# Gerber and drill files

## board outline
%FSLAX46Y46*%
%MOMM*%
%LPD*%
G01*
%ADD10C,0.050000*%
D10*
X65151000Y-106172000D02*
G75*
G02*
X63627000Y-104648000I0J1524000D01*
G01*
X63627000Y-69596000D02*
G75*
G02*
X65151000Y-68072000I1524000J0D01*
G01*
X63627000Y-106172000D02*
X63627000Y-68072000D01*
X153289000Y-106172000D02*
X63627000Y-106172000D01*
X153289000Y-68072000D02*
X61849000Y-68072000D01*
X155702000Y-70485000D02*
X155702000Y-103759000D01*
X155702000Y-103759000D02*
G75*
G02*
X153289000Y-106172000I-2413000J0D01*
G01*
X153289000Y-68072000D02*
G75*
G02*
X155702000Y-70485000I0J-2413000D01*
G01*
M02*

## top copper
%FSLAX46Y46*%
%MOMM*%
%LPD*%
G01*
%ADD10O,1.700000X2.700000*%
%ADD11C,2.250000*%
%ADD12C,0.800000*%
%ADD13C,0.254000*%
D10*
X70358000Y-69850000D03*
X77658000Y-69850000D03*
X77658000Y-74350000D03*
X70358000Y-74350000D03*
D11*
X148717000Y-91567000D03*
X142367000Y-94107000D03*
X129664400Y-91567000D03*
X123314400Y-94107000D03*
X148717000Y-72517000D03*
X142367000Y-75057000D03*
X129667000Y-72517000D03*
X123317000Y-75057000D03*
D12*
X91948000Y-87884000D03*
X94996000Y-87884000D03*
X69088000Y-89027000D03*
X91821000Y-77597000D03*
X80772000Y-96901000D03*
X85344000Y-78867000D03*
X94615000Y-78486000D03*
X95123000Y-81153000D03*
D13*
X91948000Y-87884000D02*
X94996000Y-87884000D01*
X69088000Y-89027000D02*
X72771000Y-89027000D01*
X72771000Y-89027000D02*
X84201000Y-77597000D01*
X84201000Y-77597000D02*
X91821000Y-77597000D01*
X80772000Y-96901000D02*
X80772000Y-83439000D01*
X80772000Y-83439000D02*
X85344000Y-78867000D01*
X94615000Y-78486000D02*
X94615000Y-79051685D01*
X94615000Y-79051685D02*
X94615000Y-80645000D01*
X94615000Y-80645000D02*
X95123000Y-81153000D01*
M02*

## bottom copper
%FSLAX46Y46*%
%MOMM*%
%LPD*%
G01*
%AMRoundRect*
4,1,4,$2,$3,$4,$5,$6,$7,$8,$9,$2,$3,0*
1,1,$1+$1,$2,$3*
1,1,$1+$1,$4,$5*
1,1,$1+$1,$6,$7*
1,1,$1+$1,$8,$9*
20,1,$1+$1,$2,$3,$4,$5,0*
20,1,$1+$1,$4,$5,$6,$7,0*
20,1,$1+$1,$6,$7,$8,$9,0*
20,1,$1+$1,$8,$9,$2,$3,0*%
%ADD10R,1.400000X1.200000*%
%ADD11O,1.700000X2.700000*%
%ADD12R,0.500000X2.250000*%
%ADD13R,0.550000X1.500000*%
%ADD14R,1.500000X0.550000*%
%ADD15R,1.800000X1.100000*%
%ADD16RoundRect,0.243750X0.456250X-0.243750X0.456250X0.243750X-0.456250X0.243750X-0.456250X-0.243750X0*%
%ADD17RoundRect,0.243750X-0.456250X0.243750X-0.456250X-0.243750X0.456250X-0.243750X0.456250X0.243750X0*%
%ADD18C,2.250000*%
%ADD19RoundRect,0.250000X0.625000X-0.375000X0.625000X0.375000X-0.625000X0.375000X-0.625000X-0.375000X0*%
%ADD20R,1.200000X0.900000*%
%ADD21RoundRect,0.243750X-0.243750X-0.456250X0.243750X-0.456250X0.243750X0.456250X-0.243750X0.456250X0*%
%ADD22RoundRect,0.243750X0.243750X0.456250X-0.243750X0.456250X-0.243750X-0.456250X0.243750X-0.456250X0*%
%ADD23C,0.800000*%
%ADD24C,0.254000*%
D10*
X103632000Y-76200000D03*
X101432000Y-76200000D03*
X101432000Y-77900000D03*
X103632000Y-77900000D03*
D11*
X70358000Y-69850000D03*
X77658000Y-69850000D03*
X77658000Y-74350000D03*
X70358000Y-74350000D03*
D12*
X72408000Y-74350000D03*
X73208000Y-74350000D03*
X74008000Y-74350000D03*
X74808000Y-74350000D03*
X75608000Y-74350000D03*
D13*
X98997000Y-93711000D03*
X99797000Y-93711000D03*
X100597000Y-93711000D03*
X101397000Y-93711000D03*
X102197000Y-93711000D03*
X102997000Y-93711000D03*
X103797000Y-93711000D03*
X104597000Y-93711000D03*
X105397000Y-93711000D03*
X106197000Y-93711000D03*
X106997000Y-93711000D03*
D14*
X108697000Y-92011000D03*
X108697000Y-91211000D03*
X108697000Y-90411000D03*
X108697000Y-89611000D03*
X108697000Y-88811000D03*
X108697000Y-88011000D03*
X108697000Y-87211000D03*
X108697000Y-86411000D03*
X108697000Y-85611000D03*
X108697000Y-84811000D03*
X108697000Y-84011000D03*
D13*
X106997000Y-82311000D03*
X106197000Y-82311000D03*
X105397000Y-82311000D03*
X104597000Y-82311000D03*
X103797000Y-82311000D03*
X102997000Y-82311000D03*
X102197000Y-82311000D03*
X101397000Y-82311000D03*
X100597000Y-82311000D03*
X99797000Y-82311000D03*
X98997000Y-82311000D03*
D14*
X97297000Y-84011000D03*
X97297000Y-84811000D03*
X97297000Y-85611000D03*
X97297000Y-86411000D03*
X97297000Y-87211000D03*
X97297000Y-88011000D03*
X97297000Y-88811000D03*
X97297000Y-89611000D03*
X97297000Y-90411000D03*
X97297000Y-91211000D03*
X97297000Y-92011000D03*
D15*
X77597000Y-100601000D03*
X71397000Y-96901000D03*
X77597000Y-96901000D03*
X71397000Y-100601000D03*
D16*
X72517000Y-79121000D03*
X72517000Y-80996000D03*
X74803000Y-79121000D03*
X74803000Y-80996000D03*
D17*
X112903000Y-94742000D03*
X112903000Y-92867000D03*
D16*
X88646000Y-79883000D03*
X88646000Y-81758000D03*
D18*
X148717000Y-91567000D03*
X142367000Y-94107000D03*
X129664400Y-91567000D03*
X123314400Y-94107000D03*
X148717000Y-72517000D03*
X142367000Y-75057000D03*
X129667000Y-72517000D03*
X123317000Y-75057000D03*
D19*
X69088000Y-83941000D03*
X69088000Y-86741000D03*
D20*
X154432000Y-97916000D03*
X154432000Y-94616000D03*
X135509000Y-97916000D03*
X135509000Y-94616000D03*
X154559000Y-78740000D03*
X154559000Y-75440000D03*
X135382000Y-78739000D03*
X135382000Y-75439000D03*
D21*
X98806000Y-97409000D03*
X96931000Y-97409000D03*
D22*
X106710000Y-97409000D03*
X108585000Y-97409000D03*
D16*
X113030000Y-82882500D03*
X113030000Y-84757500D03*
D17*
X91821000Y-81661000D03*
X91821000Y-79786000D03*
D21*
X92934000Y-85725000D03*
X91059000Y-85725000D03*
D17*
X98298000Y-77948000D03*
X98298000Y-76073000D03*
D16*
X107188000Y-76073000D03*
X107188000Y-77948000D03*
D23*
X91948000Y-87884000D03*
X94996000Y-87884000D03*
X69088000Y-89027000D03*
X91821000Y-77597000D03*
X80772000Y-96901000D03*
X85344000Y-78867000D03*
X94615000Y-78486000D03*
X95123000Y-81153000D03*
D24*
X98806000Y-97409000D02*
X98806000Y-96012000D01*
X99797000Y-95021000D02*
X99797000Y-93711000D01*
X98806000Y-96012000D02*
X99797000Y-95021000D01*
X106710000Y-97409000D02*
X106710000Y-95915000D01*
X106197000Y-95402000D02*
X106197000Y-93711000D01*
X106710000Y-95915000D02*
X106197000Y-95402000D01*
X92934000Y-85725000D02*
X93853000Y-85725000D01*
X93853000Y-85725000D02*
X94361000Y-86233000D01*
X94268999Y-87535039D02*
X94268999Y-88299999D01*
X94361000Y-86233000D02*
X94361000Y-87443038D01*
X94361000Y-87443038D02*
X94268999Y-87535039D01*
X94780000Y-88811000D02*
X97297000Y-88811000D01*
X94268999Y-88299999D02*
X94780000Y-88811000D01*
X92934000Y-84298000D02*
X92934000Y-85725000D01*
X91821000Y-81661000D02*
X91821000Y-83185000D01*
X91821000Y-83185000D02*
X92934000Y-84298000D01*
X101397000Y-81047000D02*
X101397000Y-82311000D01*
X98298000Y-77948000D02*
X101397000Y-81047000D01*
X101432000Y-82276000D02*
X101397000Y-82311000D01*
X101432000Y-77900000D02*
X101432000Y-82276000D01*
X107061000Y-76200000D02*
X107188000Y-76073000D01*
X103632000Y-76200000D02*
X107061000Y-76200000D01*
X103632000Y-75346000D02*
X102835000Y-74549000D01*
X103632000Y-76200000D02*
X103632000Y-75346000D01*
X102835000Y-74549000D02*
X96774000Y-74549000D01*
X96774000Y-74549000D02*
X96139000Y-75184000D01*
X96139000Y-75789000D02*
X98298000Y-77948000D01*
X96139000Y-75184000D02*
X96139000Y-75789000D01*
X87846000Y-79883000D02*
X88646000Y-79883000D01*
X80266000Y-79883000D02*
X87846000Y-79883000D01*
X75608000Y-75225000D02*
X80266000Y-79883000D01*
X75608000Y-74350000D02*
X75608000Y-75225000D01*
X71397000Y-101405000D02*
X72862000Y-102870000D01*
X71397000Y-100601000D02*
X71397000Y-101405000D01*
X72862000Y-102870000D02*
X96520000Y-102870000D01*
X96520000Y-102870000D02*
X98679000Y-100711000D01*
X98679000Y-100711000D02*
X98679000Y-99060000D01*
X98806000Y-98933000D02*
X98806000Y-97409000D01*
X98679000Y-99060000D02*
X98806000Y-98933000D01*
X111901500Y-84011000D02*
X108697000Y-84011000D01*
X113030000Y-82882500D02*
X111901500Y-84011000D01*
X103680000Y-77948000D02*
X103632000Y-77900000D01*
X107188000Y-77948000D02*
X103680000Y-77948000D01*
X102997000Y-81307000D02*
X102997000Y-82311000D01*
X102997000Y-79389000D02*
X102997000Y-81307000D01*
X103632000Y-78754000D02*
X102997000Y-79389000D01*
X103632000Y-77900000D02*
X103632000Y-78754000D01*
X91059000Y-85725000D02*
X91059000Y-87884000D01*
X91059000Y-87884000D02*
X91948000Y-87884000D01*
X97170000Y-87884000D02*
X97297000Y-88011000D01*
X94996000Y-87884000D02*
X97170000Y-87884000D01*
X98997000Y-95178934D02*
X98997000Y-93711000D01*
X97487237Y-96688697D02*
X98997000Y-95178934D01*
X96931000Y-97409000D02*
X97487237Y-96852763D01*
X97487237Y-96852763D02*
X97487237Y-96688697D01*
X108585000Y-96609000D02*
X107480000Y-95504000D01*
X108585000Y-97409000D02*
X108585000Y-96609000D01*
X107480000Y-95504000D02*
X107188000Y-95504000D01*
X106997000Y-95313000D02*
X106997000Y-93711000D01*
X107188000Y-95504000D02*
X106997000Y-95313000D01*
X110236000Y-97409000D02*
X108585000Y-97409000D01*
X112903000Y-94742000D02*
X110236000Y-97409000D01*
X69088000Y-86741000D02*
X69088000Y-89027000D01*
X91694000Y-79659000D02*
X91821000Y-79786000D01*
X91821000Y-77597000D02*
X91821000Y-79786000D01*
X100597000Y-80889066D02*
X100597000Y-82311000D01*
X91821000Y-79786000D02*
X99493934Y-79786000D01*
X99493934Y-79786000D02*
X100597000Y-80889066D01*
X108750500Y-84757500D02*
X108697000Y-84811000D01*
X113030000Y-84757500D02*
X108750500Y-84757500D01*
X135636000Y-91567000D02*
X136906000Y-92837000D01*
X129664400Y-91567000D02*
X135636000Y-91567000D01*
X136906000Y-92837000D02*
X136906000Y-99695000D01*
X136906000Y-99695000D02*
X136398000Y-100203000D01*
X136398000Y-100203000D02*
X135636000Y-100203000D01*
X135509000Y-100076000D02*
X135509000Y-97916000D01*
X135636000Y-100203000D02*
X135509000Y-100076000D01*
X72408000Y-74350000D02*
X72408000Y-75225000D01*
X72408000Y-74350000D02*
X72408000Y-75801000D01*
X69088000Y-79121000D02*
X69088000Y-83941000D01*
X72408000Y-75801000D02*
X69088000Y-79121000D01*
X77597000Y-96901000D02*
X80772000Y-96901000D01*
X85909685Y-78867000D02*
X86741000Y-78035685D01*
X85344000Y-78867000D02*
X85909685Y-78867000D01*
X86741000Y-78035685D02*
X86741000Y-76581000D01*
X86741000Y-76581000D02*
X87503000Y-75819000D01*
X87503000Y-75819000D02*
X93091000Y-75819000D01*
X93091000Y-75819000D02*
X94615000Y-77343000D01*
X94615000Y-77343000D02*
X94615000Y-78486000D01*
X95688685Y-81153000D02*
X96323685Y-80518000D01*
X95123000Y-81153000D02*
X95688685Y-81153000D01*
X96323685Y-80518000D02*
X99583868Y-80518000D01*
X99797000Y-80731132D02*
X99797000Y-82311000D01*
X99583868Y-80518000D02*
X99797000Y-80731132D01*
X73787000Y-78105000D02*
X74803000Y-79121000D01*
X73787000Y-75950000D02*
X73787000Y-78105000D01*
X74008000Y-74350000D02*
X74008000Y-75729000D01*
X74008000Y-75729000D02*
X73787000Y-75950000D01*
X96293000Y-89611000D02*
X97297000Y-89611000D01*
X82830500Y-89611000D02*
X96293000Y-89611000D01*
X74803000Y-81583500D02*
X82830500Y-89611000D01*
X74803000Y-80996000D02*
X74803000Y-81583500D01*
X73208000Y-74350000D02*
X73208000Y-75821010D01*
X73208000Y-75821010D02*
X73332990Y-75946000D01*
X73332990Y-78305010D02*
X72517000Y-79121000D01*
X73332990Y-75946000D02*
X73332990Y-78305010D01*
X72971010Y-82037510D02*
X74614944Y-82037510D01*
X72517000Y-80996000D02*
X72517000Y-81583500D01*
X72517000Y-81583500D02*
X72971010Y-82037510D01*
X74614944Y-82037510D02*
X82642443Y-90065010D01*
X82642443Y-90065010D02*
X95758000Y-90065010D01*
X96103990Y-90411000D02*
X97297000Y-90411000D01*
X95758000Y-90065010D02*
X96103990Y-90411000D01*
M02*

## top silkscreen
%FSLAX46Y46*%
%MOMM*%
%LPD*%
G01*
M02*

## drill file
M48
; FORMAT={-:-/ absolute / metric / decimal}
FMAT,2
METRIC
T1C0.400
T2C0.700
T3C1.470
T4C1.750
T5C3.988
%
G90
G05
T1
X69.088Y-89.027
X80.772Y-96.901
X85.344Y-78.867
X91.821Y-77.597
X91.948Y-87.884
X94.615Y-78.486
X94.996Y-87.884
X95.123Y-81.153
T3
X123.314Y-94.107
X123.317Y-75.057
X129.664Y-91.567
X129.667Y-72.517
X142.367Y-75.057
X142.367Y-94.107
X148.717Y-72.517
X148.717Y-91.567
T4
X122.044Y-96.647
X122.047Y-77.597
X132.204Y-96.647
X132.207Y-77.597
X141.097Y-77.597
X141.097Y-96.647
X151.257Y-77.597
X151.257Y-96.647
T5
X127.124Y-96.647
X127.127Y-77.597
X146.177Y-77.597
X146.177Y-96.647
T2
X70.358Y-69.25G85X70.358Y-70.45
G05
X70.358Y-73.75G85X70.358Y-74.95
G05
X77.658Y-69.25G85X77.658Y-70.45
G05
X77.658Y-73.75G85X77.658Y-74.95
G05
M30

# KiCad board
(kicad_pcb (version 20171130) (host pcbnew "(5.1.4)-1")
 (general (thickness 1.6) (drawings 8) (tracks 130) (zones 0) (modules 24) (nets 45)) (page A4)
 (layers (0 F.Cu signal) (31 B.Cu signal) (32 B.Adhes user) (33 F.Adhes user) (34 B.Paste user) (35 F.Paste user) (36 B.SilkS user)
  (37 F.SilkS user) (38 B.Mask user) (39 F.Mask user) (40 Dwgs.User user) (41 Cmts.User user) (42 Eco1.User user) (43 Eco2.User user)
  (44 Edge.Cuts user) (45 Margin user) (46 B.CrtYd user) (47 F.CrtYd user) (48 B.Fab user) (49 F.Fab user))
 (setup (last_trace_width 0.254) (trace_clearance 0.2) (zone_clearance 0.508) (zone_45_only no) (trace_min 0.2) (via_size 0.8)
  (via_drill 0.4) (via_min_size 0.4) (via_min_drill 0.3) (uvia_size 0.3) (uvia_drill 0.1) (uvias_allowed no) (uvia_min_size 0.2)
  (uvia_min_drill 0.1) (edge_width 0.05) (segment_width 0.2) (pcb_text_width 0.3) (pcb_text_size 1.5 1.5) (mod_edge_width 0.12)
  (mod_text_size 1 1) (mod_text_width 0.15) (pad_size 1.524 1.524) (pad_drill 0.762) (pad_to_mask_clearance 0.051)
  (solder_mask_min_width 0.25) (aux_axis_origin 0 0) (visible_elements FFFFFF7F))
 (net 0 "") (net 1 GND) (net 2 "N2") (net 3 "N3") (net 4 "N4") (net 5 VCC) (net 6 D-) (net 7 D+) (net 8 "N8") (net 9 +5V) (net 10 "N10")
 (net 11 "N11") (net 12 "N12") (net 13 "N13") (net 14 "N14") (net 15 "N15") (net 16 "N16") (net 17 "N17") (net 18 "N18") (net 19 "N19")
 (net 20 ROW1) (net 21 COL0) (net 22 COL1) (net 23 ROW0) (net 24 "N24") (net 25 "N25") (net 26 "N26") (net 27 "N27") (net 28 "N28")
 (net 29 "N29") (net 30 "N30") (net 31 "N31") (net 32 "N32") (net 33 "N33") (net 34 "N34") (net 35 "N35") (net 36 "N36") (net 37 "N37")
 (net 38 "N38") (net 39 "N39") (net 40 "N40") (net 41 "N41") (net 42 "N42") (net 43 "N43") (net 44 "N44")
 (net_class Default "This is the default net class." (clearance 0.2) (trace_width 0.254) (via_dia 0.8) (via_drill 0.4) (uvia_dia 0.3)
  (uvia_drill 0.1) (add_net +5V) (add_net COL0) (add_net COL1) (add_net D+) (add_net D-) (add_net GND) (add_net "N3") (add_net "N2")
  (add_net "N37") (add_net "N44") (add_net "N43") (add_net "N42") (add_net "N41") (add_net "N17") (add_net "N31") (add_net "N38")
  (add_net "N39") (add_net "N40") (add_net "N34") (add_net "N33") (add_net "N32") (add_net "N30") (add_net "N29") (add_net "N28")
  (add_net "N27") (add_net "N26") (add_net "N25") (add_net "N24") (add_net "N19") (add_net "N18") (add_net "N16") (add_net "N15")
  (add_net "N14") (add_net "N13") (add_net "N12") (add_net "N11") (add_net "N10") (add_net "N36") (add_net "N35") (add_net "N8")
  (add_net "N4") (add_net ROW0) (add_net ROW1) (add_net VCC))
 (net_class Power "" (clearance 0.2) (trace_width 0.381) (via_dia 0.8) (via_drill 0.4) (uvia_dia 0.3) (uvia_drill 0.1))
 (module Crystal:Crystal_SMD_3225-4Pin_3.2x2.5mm (layer B.Cu) (at 102.532 77.05 180)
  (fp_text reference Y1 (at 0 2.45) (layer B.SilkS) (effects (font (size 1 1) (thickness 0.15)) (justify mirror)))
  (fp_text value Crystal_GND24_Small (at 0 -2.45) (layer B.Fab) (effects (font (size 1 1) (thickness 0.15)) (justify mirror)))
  (pad 4 smd rect (at -1.1 0.85 180) (size 1.4 1.2) (layers B.Cu B.Paste B.Mask) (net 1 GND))
  (pad 3 smd rect (at 1.1 0.85 180) (size 1.4 1.2) (layers B.Cu B.Paste B.Mask) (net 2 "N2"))
  (pad 2 smd rect (at 1.1 -0.85 180) (size 1.4 1.2) (layers B.Cu B.Paste B.Mask) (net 1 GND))
  (pad 1 smd rect (at -1.1 -0.85 180) (size 1.4 1.2) (layers B.Cu B.Paste B.Mask) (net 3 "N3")))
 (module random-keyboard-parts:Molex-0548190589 (layer B.Cu) (at 74.008 69.85 270)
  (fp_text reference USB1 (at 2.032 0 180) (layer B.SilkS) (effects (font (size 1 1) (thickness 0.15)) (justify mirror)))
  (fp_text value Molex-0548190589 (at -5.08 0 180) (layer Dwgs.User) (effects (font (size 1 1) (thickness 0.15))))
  (pad 6 thru_hole oval (at 0 3.65 270) (size 2.7 1.7) (drill oval 1.9 0.7) (layers *.Cu *.Mask) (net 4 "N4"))
  (pad 6 thru_hole oval (at 0 -3.65 270) (size 2.7 1.7) (drill oval 1.9 0.7) (layers *.Cu *.Mask) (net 4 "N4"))
  (pad 6 thru_hole oval (at 4.5 -3.65 270) (size 2.7 1.7) (drill oval 1.9 0.7) (layers *.Cu *.Mask) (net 4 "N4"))
  (pad 6 thru_hole oval (at 4.5 3.65 270) (size 2.7 1.7) (drill oval 1.9 0.7) (layers *.Cu *.Mask) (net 4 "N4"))
  (pad 5 smd rect (at 4.5 1.6 270) (size 2.25 0.5) (layers B.Cu B.Paste B.Mask) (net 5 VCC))
  (pad 4 smd rect (at 4.5 0.8 270) (size 2.25 0.5) (layers B.Cu B.Paste B.Mask) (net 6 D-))
  (pad 3 smd rect (at 4.5 0 270) (size 2.25 0.5) (layers B.Cu B.Paste B.Mask) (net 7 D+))
  (pad 2 smd rect (at 4.5 -0.8 270) (size 2.25 0.5) (layers B.Cu B.Paste B.Mask) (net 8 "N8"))
  (pad 1 smd rect (at 4.5 -1.6 270) (size 2.25 0.5) (layers B.Cu B.Paste B.Mask) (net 1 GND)))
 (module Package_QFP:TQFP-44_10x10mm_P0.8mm (layer B.Cu) (at 102.997 88.011)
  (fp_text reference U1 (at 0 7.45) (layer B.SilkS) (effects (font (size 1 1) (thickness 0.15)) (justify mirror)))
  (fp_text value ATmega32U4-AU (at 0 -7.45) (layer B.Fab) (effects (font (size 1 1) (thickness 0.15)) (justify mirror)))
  (pad 44 smd rect (at -4 5.7 270) (size 1.5 0.55) (layers B.Cu B.Paste B.Mask) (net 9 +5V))
  (pad 43 smd rect (at -3.2 5.7 270) (size 1.5 0.55) (layers B.Cu B.Paste B.Mask) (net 1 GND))
  (pad 42 smd rect (at -2.4 5.7 270) (size 1.5 0.55) (layers B.Cu B.Paste B.Mask) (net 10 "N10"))
  (pad 41 smd rect (at -1.6 5.7 270) (size 1.5 0.55) (layers B.Cu B.Paste B.Mask) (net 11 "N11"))
  (pad 40 smd rect (at -0.8 5.7 270) (size 1.5 0.55) (layers B.Cu B.Paste B.Mask) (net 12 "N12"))
  (pad 39 smd rect (at 0 5.7 270) (size 1.5 0.55) (layers B.Cu B.Paste B.Mask) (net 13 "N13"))
  (pad 38 smd rect (at 0.8 5.7 270) (size 1.5 0.55) (layers B.Cu B.Paste B.Mask) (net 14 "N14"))
  (pad 37 smd rect (at 1.6 5.7 270) (size 1.5 0.55) (layers B.Cu B.Paste B.Mask) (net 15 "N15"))
  (pad 36 smd rect (at 2.4 5.7 270) (size 1.5 0.55) (layers B.Cu B.Paste B.Mask) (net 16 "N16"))
  (pad 35 smd rect (at 3.2 5.7 270) (size 1.5 0.55) (layers B.Cu B.Paste B.Mask) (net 1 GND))
  (pad 34 smd rect (at 4 5.7 270) (size 1.5 0.55) (layers B.Cu B.Paste B.Mask) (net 9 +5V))
  (pad 33 smd rect (at 5.7 4) (size 1.5 0.55) (layers B.Cu B.Paste B.Mask) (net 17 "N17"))
  (pad 32 smd rect (at 5.7 3.2) (size 1.5 0.55) (layers B.Cu B.Paste B.Mask) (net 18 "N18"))
  (pad 31 smd rect (at 5.7 2.4) (size 1.5 0.55) (layers B.Cu B.Paste B.Mask) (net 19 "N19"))
  (pad 30 smd rect (at 5.7 1.6) (size 1.5 0.55) (layers B.Cu B.Paste B.Mask) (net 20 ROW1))
  (pad 29 smd rect (at 5.7 0.8) (size 1.5 0.55) (layers B.Cu B.Paste B.Mask) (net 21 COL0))
  (pad 28 smd rect (at 5.7 0) (size 1.5 0.55) (layers B.Cu B.Paste B.Mask) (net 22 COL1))
  (pad 27 smd rect (at 5.7 -0.8) (size 1.5 0.55) (layers B.Cu B.Paste B.Mask) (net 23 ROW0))
  (pad 26 smd rect (at 5.7 -1.6) (size 1.5 0.55) (layers B.Cu B.Paste B.Mask) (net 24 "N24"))
  (pad 25 smd rect (at 5.7 -2.4) (size 1.5 0.55) (layers B.Cu B.Paste B.Mask) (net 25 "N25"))
  (pad 24 smd rect (at 5.7 -3.2) (size 1.5 0.55) (layers B.Cu B.Paste B.Mask) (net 9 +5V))
  (pad 23 smd rect (at 5.7 -4) (size 1.5 0.55) (layers B.Cu B.Paste B.Mask) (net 1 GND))
  (pad 22 smd rect (at 4 -5.7 270) (size 1.5 0.55) (layers B.Cu B.Paste B.Mask) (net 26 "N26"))
  (pad 21 smd rect (at 3.2 -5.7 270) (size 1.5 0.55) (layers B.Cu B.Paste B.Mask) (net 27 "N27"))
  (pad 20 smd rect (at 2.4 -5.7 270) (size 1.5 0.55) (layers B.Cu B.Paste B.Mask) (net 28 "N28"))
  (pad 19 smd rect (at 1.6 -5.7 270) (size 1.5 0.55) (layers B.Cu B.Paste B.Mask) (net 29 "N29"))
  (pad 18 smd rect (at 0.8 -5.7 270) (size 1.5 0.55) (layers B.Cu B.Paste B.Mask) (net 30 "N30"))
  (pad 17 smd rect (at 0 -5.7 270) (size 1.5 0.55) (layers B.Cu B.Paste B.Mask) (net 3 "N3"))
  (pad 16 smd rect (at -0.8 -5.7 270) (size 1.5 0.55) (layers B.Cu B.Paste B.Mask) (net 2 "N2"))
  (pad 15 smd rect (at -1.6 -5.7 270) (size 1.5 0.55) (layers B.Cu B.Paste B.Mask) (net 1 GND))
  (pad 14 smd rect (at -2.4 -5.7 270) (size 1.5 0.55) (layers B.Cu B.Paste B.Mask) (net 9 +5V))
  (pad 13 smd rect (at -3.2 -5.7 270) (size 1.5 0.55) (layers B.Cu B.Paste B.Mask) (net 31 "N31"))
  (pad 12 smd rect (at -4 -5.7 270) (size 1.5 0.55) (layers B.Cu B.Paste B.Mask) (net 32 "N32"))
  (pad 11 smd rect (at -5.7 -4) (size 1.5 0.55) (layers B.Cu B.Paste B.Mask) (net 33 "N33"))
  (pad 10 smd rect (at -5.7 -3.2) (size 1.5 0.55) (layers B.Cu B.Paste B.Mask) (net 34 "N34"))
  (pad 9 smd rect (at -5.7 -2.4) (size 1.5 0.55) (layers B.Cu B.Paste B.Mask) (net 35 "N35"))
  (pad 8 smd rect (at -5.7 -1.6) (size 1.5 0.55) (layers B.Cu B.Paste B.Mask) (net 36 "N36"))
  (pad 7 smd rect (at -5.7 -0.8) (size 1.5 0.55) (layers B.Cu B.Paste B.Mask) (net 9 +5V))
  (pad 6 smd rect (at -5.7 0) (size 1.5 0.55) (layers B.Cu B.Paste B.Mask) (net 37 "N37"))
  (pad 5 smd rect (at -5.7 0.8) (size 1.5 0.55) (layers B.Cu B.Paste B.Mask) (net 1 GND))
  (pad 4 smd rect (at -5.7 1.6) (size 1.5 0.55) (layers B.Cu B.Paste B.Mask) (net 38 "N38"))
  (pad 3 smd rect (at -5.7 2.4) (size 1.5 0.55) (layers B.Cu B.Paste B.Mask) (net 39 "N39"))
  (pad 2 smd rect (at -5.7 3.2) (size 1.5 0.55) (layers B.Cu B.Paste B.Mask) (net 9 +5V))
  (pad 1 smd rect (at -5.7 4) (size 1.5 0.55) (layers B.Cu B.Paste B.Mask) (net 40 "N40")))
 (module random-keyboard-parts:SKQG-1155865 (layer B.Cu) (at 74.497 98.751 180)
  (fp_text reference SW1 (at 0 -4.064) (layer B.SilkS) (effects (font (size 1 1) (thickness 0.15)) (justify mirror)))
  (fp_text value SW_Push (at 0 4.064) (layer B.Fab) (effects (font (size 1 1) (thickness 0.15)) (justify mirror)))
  (pad 4 smd rect (at -3.1 -1.85 180) (size 1.8 1.1) (layers B.Cu B.Paste B.Mask))
  (pad 3 smd rect (at 3.1 1.85 180) (size 1.8 1.1) (layers B.Cu B.Paste B.Mask))
  (pad 2 smd rect (at -3.1 1.85 180) (size 1.8 1.1) (layers B.Cu B.Paste B.Mask) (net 31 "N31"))
  (pad 1 smd rect (at 3.1 -1.85 180) (size 1.8 1.1) (layers B.Cu B.Paste B.Mask) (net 1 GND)))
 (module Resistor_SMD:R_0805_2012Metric (layer B.Cu) (at 72.517 80.0585 90)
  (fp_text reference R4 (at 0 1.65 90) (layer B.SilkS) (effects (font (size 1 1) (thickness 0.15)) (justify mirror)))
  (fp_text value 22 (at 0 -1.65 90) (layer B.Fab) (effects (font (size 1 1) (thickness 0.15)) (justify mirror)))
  (pad 2 smd roundrect (at 0.9375 0 90) (size 0.975 1.4) (layers B.Cu B.Paste B.Mask) (roundrect_rratio 0.25) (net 6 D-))
  (pad 1 smd roundrect (at -0.9375 0 90) (size 0.975 1.4) (layers B.Cu B.Paste B.Mask) (roundrect_rratio 0.25) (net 39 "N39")))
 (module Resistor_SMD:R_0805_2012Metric (layer B.Cu) (at 74.803 80.0585 90)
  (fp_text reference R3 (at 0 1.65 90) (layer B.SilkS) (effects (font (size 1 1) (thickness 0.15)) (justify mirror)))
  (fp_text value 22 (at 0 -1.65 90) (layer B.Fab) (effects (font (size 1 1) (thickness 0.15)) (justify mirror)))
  (pad 2 smd roundrect (at 0.9375 0 90) (size 0.975 1.4) (layers B.Cu B.Paste B.Mask) (roundrect_rratio 0.25) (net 7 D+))
  (pad 1 smd roundrect (at -0.9375 0 90) (size 0.975 1.4) (layers B.Cu B.Paste B.Mask) (roundrect_rratio 0.25) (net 38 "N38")))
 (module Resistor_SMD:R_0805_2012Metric (layer B.Cu) (at 112.903 93.8045 270)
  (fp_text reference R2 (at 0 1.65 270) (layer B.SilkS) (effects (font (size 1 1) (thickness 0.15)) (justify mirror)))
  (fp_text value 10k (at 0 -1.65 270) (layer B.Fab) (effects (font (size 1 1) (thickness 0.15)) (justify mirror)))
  (pad 2 smd roundrect (at 0.9375 0 270) (size 0.975 1.4) (layers B.Cu B.Paste B.Mask) (roundrect_rratio 0.25) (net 9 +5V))
  (pad 1 smd roundrect (at -0.9375 0 270) (size 0.975 1.4) (layers B.Cu B.Paste B.Mask) (roundrect_rratio 0.25) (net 31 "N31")))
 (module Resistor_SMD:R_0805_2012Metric (layer B.Cu) (at 88.646 80.8205 90)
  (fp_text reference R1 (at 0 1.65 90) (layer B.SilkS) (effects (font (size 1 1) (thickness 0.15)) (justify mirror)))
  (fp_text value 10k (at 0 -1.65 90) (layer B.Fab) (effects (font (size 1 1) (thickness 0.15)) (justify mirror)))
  (pad 2 smd roundrect (at 0.9375 0 90) (size 0.975 1.4) (layers B.Cu B.Paste B.Mask) (roundrect_rratio 0.25) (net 1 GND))
  (pad 1 smd roundrect (at -0.9375 0 90) (size 0.975 1.4) (layers B.Cu B.Paste B.Mask) (roundrect_rratio 0.25) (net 17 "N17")))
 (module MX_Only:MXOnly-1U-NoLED (layer F.Cu) (at 146.177 96.647)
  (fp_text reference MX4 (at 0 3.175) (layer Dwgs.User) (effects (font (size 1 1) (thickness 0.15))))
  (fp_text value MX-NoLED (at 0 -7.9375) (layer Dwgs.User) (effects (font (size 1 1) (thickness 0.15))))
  (pad 2 thru_hole circle (at 2.54 -5.08) (size 2.25 2.25) (drill 1.47) (layers *.Cu B.Mask) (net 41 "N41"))
  (pad "" np_thru_hole circle (at 0 0) (size 3.9878 3.9878) (drill 3.9878) (layers *.Cu *.Mask))
  (pad 1 thru_hole circle (at -3.81 -2.54) (size 2.25 2.25) (drill 1.47) (layers *.Cu B.Mask) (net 22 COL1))
  (pad "" np_thru_hole circle (at -5.08 0 48.0996) (size 1.75 1.75) (drill 1.75) (layers *.Cu *.Mask))
  (pad "" np_thru_hole circle (at 5.08 0 48.0996) (size 1.75 1.75) (drill 1.75) (layers *.Cu *.Mask)))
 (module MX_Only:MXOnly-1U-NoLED (layer F.Cu) (at 127.1244 96.647)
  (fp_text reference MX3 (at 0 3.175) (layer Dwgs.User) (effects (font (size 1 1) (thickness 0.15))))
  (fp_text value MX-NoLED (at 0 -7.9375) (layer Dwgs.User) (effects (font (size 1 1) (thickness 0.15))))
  (pad 2 thru_hole circle (at 2.54 -5.08) (size 2.25 2.25) (drill 1.47) (layers *.Cu B.Mask) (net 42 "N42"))
  (pad "" np_thru_hole circle (at 0 0) (size 3.9878 3.9878) (drill 3.9878) (layers *.Cu *.Mask))
  (pad 1 thru_hole circle (at -3.81 -2.54) (size 2.25 2.25) (drill 1.47) (layers *.Cu B.Mask) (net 21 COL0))
  (pad "" np_thru_hole circle (at -5.08 0 48.0996) (size 1.75 1.75) (drill 1.75) (layers *.Cu *.Mask))
  (pad "" np_thru_hole circle (at 5.08 0 48.0996) (size 1.75 1.75) (drill 1.75) (layers *.Cu *.Mask)))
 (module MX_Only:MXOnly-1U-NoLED (layer F.Cu) (at 146.177 77.597)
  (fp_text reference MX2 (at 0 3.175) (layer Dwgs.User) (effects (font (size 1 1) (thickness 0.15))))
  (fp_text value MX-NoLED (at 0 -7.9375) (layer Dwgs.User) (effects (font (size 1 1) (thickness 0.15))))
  (pad 2 thru_hole circle (at 2.54 -5.08) (size 2.25 2.25) (drill 1.47) (layers *.Cu B.Mask) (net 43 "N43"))
  (pad "" np_thru_hole circle (at 0 0) (size 3.9878 3.9878) (drill 3.9878) (layers *.Cu *.Mask))
  (pad 1 thru_hole circle (at -3.81 -2.54) (size 2.25 2.25) (drill 1.47) (layers *.Cu B.Mask) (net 22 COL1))
  (pad "" np_thru_hole circle (at -5.08 0 48.0996) (size 1.75 1.75) (drill 1.75) (layers *.Cu *.Mask))
  (pad "" np_thru_hole circle (at 5.08 0 48.0996) (size 1.75 1.75) (drill 1.75) (layers *.Cu *.Mask)))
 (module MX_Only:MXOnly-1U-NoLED (layer F.Cu) (at 127.127 77.597)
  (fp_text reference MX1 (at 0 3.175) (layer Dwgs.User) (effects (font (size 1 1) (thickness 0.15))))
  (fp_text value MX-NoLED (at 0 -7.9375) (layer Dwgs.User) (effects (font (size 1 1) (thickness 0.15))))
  (pad 2 thru_hole circle (at 2.54 -5.08) (size 2.25 2.25) (drill 1.47) (layers *.Cu B.Mask) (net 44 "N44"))
  (pad "" np_thru_hole circle (at 0 0) (size 3.9878 3.9878) (drill 3.9878) (layers *.Cu *.Mask))
  (pad 1 thru_hole circle (at -3.81 -2.54) (size 2.25 2.25) (drill 1.47) (layers *.Cu B.Mask) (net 21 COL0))
  (pad "" np_thru_hole circle (at -5.08 0 48.0996) (size 1.75 1.75) (drill 1.75) (layers *.Cu *.Mask))
  (pad "" np_thru_hole circle (at 5.08 0 48.0996) (size 1.75 1.75) (drill 1.75) (layers *.Cu *.Mask)))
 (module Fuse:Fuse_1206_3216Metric (layer B.Cu) (at 69.088 85.341 90)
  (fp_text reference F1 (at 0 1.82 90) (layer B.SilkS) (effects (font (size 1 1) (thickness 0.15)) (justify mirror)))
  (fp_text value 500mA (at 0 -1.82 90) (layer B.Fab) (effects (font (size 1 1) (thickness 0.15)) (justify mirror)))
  (pad 2 smd roundrect (at 1.4 0 90) (size 1.25 1.75) (layers B.Cu B.Paste B.Mask) (roundrect_rratio 0.2) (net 5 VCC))
  (pad 1 smd roundrect (at -1.4 0 90) (size 1.25 1.75) (layers B.Cu B.Paste B.Mask) (roundrect_rratio 0.2) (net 9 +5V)))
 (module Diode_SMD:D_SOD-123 (layer B.Cu) (at 154.432 96.266 270)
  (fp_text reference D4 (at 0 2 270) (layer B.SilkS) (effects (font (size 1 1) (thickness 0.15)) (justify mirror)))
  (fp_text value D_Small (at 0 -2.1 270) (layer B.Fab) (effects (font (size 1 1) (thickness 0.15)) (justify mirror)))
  (pad 2 smd rect (at 1.65 0 270) (size 0.9 1.2) (layers B.Cu B.Paste B.Mask) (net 41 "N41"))
  (pad 1 smd rect (at -1.65 0 270) (size 0.9 1.2) (layers B.Cu B.Paste B.Mask) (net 20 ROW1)))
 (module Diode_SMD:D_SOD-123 (layer B.Cu) (at 135.509 96.266 270)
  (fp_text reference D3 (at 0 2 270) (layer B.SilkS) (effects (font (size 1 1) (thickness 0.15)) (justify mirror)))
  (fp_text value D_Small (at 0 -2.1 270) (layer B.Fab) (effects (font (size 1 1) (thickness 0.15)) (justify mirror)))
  (pad 2 smd rect (at 1.65 0 270) (size 0.9 1.2) (layers B.Cu B.Paste B.Mask) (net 42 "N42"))
  (pad 1 smd rect (at -1.65 0 270) (size 0.9 1.2) (layers B.Cu B.Paste B.Mask) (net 20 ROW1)))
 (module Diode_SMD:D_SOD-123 (layer B.Cu) (at 154.559 77.09 270)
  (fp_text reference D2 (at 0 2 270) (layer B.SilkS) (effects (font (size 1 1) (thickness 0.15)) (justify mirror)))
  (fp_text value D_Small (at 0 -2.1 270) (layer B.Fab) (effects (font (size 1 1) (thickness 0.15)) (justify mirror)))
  (pad 2 smd rect (at 1.65 0 270) (size 0.9 1.2) (layers B.Cu B.Paste B.Mask) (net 43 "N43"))
  (pad 1 smd rect (at -1.65 0 270) (size 0.9 1.2) (layers B.Cu B.Paste B.Mask) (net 23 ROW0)))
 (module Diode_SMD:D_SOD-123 (layer B.Cu) (at 135.382 77.089 270)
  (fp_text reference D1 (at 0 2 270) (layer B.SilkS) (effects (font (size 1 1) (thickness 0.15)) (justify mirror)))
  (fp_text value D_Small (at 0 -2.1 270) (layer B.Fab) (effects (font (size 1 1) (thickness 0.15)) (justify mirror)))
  (pad 2 smd rect (at 1.65 0 270) (size 0.9 1.2) (layers B.Cu B.Paste B.Mask) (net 44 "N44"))
  (pad 1 smd rect (at -1.65 0 270) (size 0.9 1.2) (layers B.Cu B.Paste B.Mask) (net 23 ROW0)))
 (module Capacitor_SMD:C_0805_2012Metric (layer B.Cu) (at 97.8685 97.409)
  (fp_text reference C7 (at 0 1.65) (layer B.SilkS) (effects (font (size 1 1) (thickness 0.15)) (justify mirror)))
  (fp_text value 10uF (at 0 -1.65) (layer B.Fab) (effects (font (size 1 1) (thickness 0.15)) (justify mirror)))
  (pad 2 smd roundrect (at 0.9375 0) (size 0.975 1.4) (layers B.Cu B.Paste B.Mask) (roundrect_rratio 0.25) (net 1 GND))
  (pad 1 smd roundrect (at -0.9375 0) (size 0.975 1.4) (layers B.Cu B.Paste B.Mask) (roundrect_rratio 0.25) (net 9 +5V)))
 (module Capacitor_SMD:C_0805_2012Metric (layer B.Cu) (at 107.6475 97.409 180)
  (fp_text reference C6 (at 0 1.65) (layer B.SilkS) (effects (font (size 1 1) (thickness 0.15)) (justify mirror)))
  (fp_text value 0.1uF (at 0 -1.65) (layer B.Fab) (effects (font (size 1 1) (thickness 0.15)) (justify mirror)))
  (pad 2 smd roundrect (at 0.9375 0 180) (size 0.975 1.4) (layers B.Cu B.Paste B.Mask) (roundrect_rratio 0.25) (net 1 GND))
  (pad 1 smd roundrect (at -0.9375 0 180) (size 0.975 1.4) (layers B.Cu B.Paste B.Mask) (roundrect_rratio 0.25) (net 9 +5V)))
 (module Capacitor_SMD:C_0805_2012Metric (layer B.Cu) (at 113.03 83.82 90)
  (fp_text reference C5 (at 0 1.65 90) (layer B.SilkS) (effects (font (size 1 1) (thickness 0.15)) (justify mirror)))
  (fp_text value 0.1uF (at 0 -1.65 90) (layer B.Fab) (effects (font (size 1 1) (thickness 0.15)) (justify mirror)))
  (pad 2 smd roundrect (at 0.9375 0 90) (size 0.975 1.4) (layers B.Cu B.Paste B.Mask) (roundrect_rratio 0.25) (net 1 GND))
  (pad 1 smd roundrect (at -0.9375 0 90) (size 0.975 1.4) (layers B.Cu B.Paste B.Mask) (roundrect_rratio 0.25) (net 9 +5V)))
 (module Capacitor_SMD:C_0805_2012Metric (layer B.Cu) (at 91.821 80.7235 270)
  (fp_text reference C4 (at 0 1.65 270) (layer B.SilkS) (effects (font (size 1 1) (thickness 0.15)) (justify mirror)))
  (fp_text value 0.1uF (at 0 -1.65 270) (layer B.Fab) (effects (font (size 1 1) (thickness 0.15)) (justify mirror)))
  (pad 2 smd roundrect (at 0.9375 0 270) (size 0.975 1.4) (layers B.Cu B.Paste B.Mask) (roundrect_rratio 0.25) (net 1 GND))
  (pad 1 smd roundrect (at -0.9375 0 270) (size 0.975 1.4) (layers B.Cu B.Paste B.Mask) (roundrect_rratio 0.25) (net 9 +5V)))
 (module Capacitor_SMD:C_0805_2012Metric (layer B.Cu) (at 91.9965 85.725)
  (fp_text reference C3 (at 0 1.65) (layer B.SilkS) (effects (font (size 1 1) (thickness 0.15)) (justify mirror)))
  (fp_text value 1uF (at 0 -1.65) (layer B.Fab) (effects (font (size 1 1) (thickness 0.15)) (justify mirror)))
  (pad 2 smd roundrect (at 0.9375 0) (size 0.975 1.4) (layers B.Cu B.Paste B.Mask) (roundrect_rratio 0.25) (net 1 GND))
  (pad 1 smd roundrect (at -0.9375 0) (size 0.975 1.4) (layers B.Cu B.Paste B.Mask) (roundrect_rratio 0.25) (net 37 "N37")))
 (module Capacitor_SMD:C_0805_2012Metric (layer B.Cu) (at 98.298 77.0105 270)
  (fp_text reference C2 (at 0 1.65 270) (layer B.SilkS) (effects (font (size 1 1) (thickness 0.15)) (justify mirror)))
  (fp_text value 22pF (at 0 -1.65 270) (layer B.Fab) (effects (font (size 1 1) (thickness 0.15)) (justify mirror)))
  (pad 2 smd roundrect (at 0.9375 0 270) (size 0.975 1.4) (layers B.Cu B.Paste B.Mask) (roundrect_rratio 0.25) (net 1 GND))
  (pad 1 smd roundrect (at -0.9375 0 270) (size 0.975 1.4) (layers B.Cu B.Paste B.Mask) (roundrect_rratio 0.25) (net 2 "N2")))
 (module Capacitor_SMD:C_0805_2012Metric (layer B.Cu) (at 107.188 77.0105 90)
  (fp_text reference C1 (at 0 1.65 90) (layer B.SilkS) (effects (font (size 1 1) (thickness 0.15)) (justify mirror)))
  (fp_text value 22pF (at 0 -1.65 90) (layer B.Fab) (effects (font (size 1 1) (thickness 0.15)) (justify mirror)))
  (pad 2 smd roundrect (at 0.9375 0 90) (size 0.975 1.4) (layers B.Cu B.Paste B.Mask) (roundrect_rratio 0.25) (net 1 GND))
  (pad 1 smd roundrect (at -0.9375 0 90) (size 0.975 1.4) (layers B.Cu B.Paste B.Mask) (roundrect_rratio 0.25) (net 3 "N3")))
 (gr_arc (start 65.151 104.648) (end 63.627 104.648) (angle -90) (layer Edge.Cuts) (width 0.05))
 (gr_arc (start 65.151 69.596) (end 65.151 68.072) (angle -90) (layer Edge.Cuts) (width 0.05))
 (gr_line (start 63.627 106.172) (end 63.627 68.072) (layer Edge.Cuts) (width 0.05))
 (gr_line (start 153.289 106.172) (end 63.627 106.172) (layer Edge.Cuts) (width 0.05))
 (gr_line (start 153.289 68.072) (end 61.849 68.072) (layer Edge.Cuts) (width 0.05))
 (gr_line (start 155.702 70.485) (end 155.702 103.759) (layer Edge.Cuts) (width 0.05))
 (gr_arc (start 153.289 103.759) (end 153.289 106.172) (angle -90) (layer Edge.Cuts) (width 0.05))
 (gr_arc (start 153.289 70.485) (end 155.702 70.485) (angle -90) (layer Edge.Cuts) (width 0.05))
 (segment (start 98.806 97.409) (end 98.806 96.012) (width 0.254) (layer B.Cu) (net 1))
 (segment (start 99.797 95.021) (end 99.797 93.711) (width 0.254) (layer B.Cu) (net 1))
 (segment (start 98.806 96.012) (end 99.797 95.021) (width 0.254) (layer B.Cu) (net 1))
 (segment (start 106.71 97.409) (end 106.71 95.915) (width 0.254) (layer B.Cu) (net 1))
 (segment (start 106.197 95.402) (end 106.197 93.711) (width 0.254) (layer B.Cu) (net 1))
 (segment (start 106.71 95.915) (end 106.197 95.402) (width 0.254) (layer B.Cu) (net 1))
 (segment (start 92.934 85.725) (end 93.853 85.725) (width 0.254) (layer B.Cu) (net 1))
 (segment (start 93.853 85.725) (end 94.361 86.233) (width 0.254) (layer B.Cu) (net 1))
 (segment (start 94.268999 87.535039) (end 94.268999 88.299999) (width 0.254) (layer B.Cu) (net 1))
 (segment (start 94.361 86.233) (end 94.361 87.443038) (width 0.254) (layer B.Cu) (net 1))
 (segment (start 94.361 87.443038) (end 94.268999 87.535039) (width 0.254) (layer B.Cu) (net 1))
 (segment (start 94.78 88.811) (end 97.297 88.811) (width 0.254) (layer B.Cu) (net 1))
 (segment (start 94.268999 88.299999) (end 94.78 88.811) (width 0.254) (layer B.Cu) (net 1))
 (segment (start 92.934 84.298) (end 92.934 85.725) (width 0.254) (layer B.Cu) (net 1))
 (segment (start 91.821 81.661) (end 91.821 83.185) (width 0.254) (layer B.Cu) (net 1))
 (segment (start 91.821 83.185) (end 92.934 84.298) (width 0.254) (layer B.Cu) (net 1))
 (segment (start 101.397 81.047) (end 101.397 82.311) (width 0.254) (layer B.Cu) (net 1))
 (segment (start 98.298 77.948) (end 101.397 81.047) (width 0.254) (layer B.Cu) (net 1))
 (segment (start 101.432 82.276) (end 101.397 82.311) (width 0.254) (layer B.Cu) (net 1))
 (segment (start 101.432 77.9) (end 101.432 82.276) (width 0.254) (layer B.Cu) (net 1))
 (segment (start 107.061 76.2) (end 107.188 76.073) (width 0.254) (layer B.Cu) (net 1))
 (segment (start 103.632 76.2) (end 107.061 76.2) (width 0.254) (layer B.Cu) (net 1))
 (segment (start 103.632 75.346) (end 102.835 74.549) (width 0.254) (layer B.Cu) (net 1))
 (segment (start 103.632 76.2) (end 103.632 75.346) (width 0.254) (layer B.Cu) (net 1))
 (segment (start 102.835 74.549) (end 96.774 74.549) (width 0.254) (layer B.Cu) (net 1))
 (segment (start 96.774 74.549) (end 96.139 75.184) (width 0.254) (layer B.Cu) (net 1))
 (segment (start 96.139 75.789) (end 98.298 77.948) (width 0.254) (layer B.Cu) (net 1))
 (segment (start 96.139 75.184) (end 96.139 75.789) (width 0.254) (layer B.Cu) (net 1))
 (segment (start 87.846 79.883) (end 88.646 79.883) (width 0.254) (layer B.Cu) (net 1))
 (segment (start 80.266 79.883) (end 87.846 79.883) (width 0.254) (layer B.Cu) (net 1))
 (segment (start 75.608 75.225) (end 80.266 79.883) (width 0.254) (layer B.Cu) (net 1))
 (segment (start 75.608 74.35) (end 75.608 75.225) (width 0.254) (layer B.Cu) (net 1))
 (segment (start 71.397 101.405) (end 72.862 102.87) (width 0.254) (layer B.Cu) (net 1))
 (segment (start 71.397 100.601) (end 71.397 101.405) (width 0.254) (layer B.Cu) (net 1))
 (segment (start 72.862 102.87) (end 96.52 102.87) (width 0.254) (layer B.Cu) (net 1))
 (segment (start 96.52 102.87) (end 98.679 100.711) (width 0.254) (layer B.Cu) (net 1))
 (segment (start 98.679 100.711) (end 98.679 99.06) (width 0.254) (layer B.Cu) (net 1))
 (segment (start 98.806 98.933) (end 98.806 97.409) (width 0.254) (layer B.Cu) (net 1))
 (segment (start 98.679 99.06) (end 98.806 98.933) (width 0.254) (layer B.Cu) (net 1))
 (segment (start 111.9015 84.011) (end 108.697 84.011) (width 0.254) (layer B.Cu) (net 1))
 (segment (start 113.03 82.8825) (end 111.9015 84.011) (width 0.254) (layer B.Cu) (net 1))
 (segment (start 103.68 77.948) (end 103.632 77.9) (width 0.254) (layer B.Cu) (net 3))
 (segment (start 107.188 77.948) (end 103.68 77.948) (width 0.254) (layer B.Cu) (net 3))
 (segment (start 102.997 81.307) (end 102.997 82.311) (width 0.254) (layer B.Cu) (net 3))
 (segment (start 102.997 79.389) (end 102.997 81.307) (width 0.254) (layer B.Cu) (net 3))
 (segment (start 103.632 78.754) (end 102.997 79.389) (width 0.254) (layer B.Cu) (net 3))
 (segment (start 103.632 77.9) (end 103.632 78.754) (width 0.254) (layer B.Cu) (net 3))
 (segment (start 91.059 85.725) (end 91.059 87.884) (width 0.254) (layer B.Cu) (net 37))
 (via (at 91.948 87.884) (size 0.8) (drill 0.4) (layers F.Cu B.Cu) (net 37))
 (segment (start 91.059 87.884) (end 91.948 87.884) (width 0.254) (layer B.Cu) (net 37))
 (via (at 94.996 87.884) (size 0.8) (drill 0.4) (layers F.Cu B.Cu) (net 37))
 (segment (start 91.948 87.884) (end 94.996 87.884) (width 0.254) (layer F.Cu) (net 37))
 (segment (start 97.17 87.884) (end 97.297 88.011) (width 0.254) (layer B.Cu) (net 37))
 (segment (start 94.996 87.884) (end 97.17 87.884) (width 0.254) (layer B.Cu) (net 37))
 (segment (start 98.997 95.178934) (end 98.997 93.711) (width 0.254) (layer B.Cu) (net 9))
 (segment (start 97.487237 96.688697) (end 98.997 95.178934) (width 0.254) (layer B.Cu) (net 9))
 (segment (start 96.931 97.409) (end 97.487237 96.852763) (width 0.254) (layer B.Cu) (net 9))
 (segment (start 97.487237 96.852763) (end 97.487237 96.688697) (width 0.254) (layer B.Cu) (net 9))
 (segment (start 108.585 96.609) (end 107.48 95.504) (width 0.254) (layer B.Cu) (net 9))
 (segment (start 108.585 97.409) (end 108.585 96.609) (width 0.254) (layer B.Cu) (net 9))
 (segment (start 107.48 95.504) (end 107.188 95.504) (width 0.254) (layer B.Cu) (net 9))
 (segment (start 106.997 95.313) (end 106.997 93.711) (width 0.254) (layer B.Cu) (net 9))
 (segment (start 107.188 95.504) (end 106.997 95.313) (width 0.254) (layer B.Cu) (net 9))
 (segment (start 110.236 97.409) (end 108.585 97.409) (width 0.254) (layer B.Cu) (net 9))
 (segment (start 112.903 94.742) (end 110.236 97.409) (width 0.254) (layer B.Cu) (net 9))
 (via (at 69.088 89.027) (size 0.8) (drill 0.4) (layers F.Cu B.Cu) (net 9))
 (segment (start 69.088 86.741) (end 69.088 89.027) (width 0.254) (layer B.Cu) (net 9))
 (segment (start 69.088 89.027) (end 72.771 89.027) (width 0.254) (layer F.Cu) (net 9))
 (segment (start 72.771 89.027) (end 84.201 77.597) (width 0.254) (layer F.Cu) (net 9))
 (segment (start 91.694 79.659) (end 91.821 79.786) (width 0.254) (layer B.Cu) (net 9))
 (via (at 91.821 77.597) (size 0.8) (drill 0.4) (layers F.Cu B.Cu) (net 9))
 (segment (start 84.201 77.597) (end 91.821 77.597) (width 0.254) (layer F.Cu) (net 9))
 (segment (start 91.821 77.597) (end 91.821 79.786) (width 0.254) (layer B.Cu) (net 9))
 (segment (start 100.597 80.889066) (end 100.597 82.311) (width 0.254) (layer B.Cu) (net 9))
 (segment (start 91.821 79.786) (end 99.493934 79.786) (width 0.254) (layer B.Cu) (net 9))
 (segment (start 99.493934 79.786) (end 100.597 80.889066) (width 0.254) (layer B.Cu) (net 9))
 (segment (start 108.7505 84.7575) (end 108.697 84.811) (width 0.254) (layer B.Cu) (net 9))
 (segment (start 113.03 84.7575) (end 108.7505 84.7575) (width 0.254) (layer B.Cu) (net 9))
 (segment (start 135.636 91.567) (end 136.906 92.837) (width 0.254) (layer B.Cu) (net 42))
 (segment (start 129.6644 91.567) (end 135.636 91.567) (width 0.254) (layer B.Cu) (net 42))
 (segment (start 136.906 92.837) (end 136.906 99.695) (width 0.254) (layer B.Cu) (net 42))
 (segment (start 136.906 99.695) (end 136.398 100.203) (width 0.254) (layer B.Cu) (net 42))
 (segment (start 136.398 100.203) (end 135.636 100.203) (width 0.254) (layer B.Cu) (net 42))
 (segment (start 135.509 100.076) (end 135.509 97.916) (width 0.254) (layer B.Cu) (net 42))
 (segment (start 135.636 100.203) (end 135.509 100.076) (width 0.254) (layer B.Cu) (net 42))
 (segment (start 72.408 74.35) (end 72.408 75.225) (width 0.254) (layer B.Cu) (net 5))
 (segment (start 72.408 74.35) (end 72.408 75.801) (width 0.254) (layer B.Cu) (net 5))
 (segment (start 69.088 79.121) (end 69.088 83.941) (width 0.254) (layer B.Cu) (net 5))
 (segment (start 72.408 75.801) (end 69.088 79.121) (width 0.254) (layer B.Cu) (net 5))
 (via (at 80.772 96.901) (size 0.8) (drill 0.4) (layers F.Cu B.Cu) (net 31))
 (segment (start 77.597 96.901) (end 80.772 96.901) (width 0.254) (layer B.Cu) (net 31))
 (via (at 85.344 78.867) (size 0.8) (drill 0.4) (layers F.Cu B.Cu) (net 31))
 (segment (start 80.772 96.901) (end 80.772 83.439) (width 0.254) (layer F.Cu) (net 31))
 (segment (start 80.772 83.439) (end 85.344 78.867) (width 0.254) (layer F.Cu) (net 31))
 (segment (start 85.909685 78.867) (end 86.741 78.035685) (width 0.254) (layer B.Cu) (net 31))
 (segment (start 85.344 78.867) (end 85.909685 78.867) (width 0.254) (layer B.Cu) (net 31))
 (segment (start 86.741 78.035685) (end 86.741 76.581) (width 0.254) (layer B.Cu) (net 31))
 (segment (start 86.741 76.581) (end 87.503 75.819) (width 0.254) (layer B.Cu) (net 31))
 (segment (start 87.503 75.819) (end 93.091 75.819) (width 0.254) (layer B.Cu) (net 31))
 (segment (start 93.091 75.819) (end 94.615 77.343) (width 0.254) (layer B.Cu) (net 31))
 (via (at 94.615 78.486) (size 0.8) (drill 0.4) (layers F.Cu B.Cu) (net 31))
 (segment (start 94.615 77.343) (end 94.615 78.486) (width 0.254) (layer B.Cu) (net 31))
 (segment (start 94.615 78.486) (end 94.615 79.051685) (width 0.254) (layer F.Cu) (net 31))
 (via (at 95.123 81.153) (size 0.8) (drill 0.4) (layers F.Cu B.Cu) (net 31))
 (segment (start 94.615 79.051685) (end 94.615 80.645) (width 0.254) (layer F.Cu) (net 31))
 (segment (start 94.615 80.645) (end 95.123 81.153) (width 0.254) (layer F.Cu) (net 31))
 (segment (start 95.688685 81.153) (end 96.323685 80.518) (width 0.254) (layer B.Cu) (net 31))
 (segment (start 95.123 81.153) (end 95.688685 81.153) (width 0.254) (layer B.Cu) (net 31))
 (segment (start 96.323685 80.518) (end 99.583868 80.518) (width 0.254) (layer B.Cu) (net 31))
 (segment (start 99.797 80.731132) (end 99.797 82.311) (width 0.254) (layer B.Cu) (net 31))
 (segment (start 99.583868 80.518) (end 99.797 80.731132) (width 0.254) (layer B.Cu) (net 31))
 (segment (start 73.787 78.105) (end 74.803 79.121) (width 0.254) (layer B.Cu) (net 7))
 (segment (start 73.787 75.95) (end 73.787 78.105) (width 0.254) (layer B.Cu) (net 7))
 (segment (start 74.008 74.35) (end 74.008 75.729) (width 0.254) (layer B.Cu) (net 7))
 (segment (start 74.008 75.729) (end 73.787 75.95) (width 0.254) (layer B.Cu) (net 7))
 (segment (start 96.293 89.611) (end 97.297 89.611) (width 0.254) (layer B.Cu) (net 38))
 (segment (start 82.8305 89.611) (end 96.293 89.611) (width 0.254) (layer B.Cu) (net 38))
 (segment (start 74.803 81.5835) (end 82.8305 89.611) (width 0.254) (layer B.Cu) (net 38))
 (segment (start 74.803 80.996) (end 74.803 81.5835) (width 0.254) (layer B.Cu) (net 38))
 (segment (start 73.208 74.35) (end 73.208 75.82101) (width 0.254) (layer B.Cu) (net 6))
 (segment (start 73.208 75.82101) (end 73.33299 75.946) (width 0.254) (layer B.Cu) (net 6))
 (segment (start 73.33299 78.30501) (end 72.517 79.121) (width 0.254) (layer B.Cu) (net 6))
 (segment (start 73.33299 75.946) (end 73.33299 78.30501) (width 0.254) (layer B.Cu) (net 6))
 (segment (start 72.97101 82.03751) (end 74.614944 82.03751) (width 0.254) (layer B.Cu) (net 39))
 (segment (start 72.517 80.996) (end 72.517 81.5835) (width 0.254) (layer B.Cu) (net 39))
 (segment (start 72.517 81.5835) (end 72.97101 82.03751) (width 0.254) (layer B.Cu) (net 39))
 (segment (start 74.614944 82.03751) (end 82.642443 90.06501) (width 0.254) (layer B.Cu) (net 39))
 (segment (start 82.642443 90.06501) (end 95.758 90.06501) (width 0.254) (layer B.Cu) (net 39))
 (segment (start 96.10399 90.411) (end 97.297 90.411) (width 0.254) (layer B.Cu) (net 39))
 (segment (start 95.758 90.06501) (end 96.10399 90.411) (width 0.254) (layer B.Cu) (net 39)))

